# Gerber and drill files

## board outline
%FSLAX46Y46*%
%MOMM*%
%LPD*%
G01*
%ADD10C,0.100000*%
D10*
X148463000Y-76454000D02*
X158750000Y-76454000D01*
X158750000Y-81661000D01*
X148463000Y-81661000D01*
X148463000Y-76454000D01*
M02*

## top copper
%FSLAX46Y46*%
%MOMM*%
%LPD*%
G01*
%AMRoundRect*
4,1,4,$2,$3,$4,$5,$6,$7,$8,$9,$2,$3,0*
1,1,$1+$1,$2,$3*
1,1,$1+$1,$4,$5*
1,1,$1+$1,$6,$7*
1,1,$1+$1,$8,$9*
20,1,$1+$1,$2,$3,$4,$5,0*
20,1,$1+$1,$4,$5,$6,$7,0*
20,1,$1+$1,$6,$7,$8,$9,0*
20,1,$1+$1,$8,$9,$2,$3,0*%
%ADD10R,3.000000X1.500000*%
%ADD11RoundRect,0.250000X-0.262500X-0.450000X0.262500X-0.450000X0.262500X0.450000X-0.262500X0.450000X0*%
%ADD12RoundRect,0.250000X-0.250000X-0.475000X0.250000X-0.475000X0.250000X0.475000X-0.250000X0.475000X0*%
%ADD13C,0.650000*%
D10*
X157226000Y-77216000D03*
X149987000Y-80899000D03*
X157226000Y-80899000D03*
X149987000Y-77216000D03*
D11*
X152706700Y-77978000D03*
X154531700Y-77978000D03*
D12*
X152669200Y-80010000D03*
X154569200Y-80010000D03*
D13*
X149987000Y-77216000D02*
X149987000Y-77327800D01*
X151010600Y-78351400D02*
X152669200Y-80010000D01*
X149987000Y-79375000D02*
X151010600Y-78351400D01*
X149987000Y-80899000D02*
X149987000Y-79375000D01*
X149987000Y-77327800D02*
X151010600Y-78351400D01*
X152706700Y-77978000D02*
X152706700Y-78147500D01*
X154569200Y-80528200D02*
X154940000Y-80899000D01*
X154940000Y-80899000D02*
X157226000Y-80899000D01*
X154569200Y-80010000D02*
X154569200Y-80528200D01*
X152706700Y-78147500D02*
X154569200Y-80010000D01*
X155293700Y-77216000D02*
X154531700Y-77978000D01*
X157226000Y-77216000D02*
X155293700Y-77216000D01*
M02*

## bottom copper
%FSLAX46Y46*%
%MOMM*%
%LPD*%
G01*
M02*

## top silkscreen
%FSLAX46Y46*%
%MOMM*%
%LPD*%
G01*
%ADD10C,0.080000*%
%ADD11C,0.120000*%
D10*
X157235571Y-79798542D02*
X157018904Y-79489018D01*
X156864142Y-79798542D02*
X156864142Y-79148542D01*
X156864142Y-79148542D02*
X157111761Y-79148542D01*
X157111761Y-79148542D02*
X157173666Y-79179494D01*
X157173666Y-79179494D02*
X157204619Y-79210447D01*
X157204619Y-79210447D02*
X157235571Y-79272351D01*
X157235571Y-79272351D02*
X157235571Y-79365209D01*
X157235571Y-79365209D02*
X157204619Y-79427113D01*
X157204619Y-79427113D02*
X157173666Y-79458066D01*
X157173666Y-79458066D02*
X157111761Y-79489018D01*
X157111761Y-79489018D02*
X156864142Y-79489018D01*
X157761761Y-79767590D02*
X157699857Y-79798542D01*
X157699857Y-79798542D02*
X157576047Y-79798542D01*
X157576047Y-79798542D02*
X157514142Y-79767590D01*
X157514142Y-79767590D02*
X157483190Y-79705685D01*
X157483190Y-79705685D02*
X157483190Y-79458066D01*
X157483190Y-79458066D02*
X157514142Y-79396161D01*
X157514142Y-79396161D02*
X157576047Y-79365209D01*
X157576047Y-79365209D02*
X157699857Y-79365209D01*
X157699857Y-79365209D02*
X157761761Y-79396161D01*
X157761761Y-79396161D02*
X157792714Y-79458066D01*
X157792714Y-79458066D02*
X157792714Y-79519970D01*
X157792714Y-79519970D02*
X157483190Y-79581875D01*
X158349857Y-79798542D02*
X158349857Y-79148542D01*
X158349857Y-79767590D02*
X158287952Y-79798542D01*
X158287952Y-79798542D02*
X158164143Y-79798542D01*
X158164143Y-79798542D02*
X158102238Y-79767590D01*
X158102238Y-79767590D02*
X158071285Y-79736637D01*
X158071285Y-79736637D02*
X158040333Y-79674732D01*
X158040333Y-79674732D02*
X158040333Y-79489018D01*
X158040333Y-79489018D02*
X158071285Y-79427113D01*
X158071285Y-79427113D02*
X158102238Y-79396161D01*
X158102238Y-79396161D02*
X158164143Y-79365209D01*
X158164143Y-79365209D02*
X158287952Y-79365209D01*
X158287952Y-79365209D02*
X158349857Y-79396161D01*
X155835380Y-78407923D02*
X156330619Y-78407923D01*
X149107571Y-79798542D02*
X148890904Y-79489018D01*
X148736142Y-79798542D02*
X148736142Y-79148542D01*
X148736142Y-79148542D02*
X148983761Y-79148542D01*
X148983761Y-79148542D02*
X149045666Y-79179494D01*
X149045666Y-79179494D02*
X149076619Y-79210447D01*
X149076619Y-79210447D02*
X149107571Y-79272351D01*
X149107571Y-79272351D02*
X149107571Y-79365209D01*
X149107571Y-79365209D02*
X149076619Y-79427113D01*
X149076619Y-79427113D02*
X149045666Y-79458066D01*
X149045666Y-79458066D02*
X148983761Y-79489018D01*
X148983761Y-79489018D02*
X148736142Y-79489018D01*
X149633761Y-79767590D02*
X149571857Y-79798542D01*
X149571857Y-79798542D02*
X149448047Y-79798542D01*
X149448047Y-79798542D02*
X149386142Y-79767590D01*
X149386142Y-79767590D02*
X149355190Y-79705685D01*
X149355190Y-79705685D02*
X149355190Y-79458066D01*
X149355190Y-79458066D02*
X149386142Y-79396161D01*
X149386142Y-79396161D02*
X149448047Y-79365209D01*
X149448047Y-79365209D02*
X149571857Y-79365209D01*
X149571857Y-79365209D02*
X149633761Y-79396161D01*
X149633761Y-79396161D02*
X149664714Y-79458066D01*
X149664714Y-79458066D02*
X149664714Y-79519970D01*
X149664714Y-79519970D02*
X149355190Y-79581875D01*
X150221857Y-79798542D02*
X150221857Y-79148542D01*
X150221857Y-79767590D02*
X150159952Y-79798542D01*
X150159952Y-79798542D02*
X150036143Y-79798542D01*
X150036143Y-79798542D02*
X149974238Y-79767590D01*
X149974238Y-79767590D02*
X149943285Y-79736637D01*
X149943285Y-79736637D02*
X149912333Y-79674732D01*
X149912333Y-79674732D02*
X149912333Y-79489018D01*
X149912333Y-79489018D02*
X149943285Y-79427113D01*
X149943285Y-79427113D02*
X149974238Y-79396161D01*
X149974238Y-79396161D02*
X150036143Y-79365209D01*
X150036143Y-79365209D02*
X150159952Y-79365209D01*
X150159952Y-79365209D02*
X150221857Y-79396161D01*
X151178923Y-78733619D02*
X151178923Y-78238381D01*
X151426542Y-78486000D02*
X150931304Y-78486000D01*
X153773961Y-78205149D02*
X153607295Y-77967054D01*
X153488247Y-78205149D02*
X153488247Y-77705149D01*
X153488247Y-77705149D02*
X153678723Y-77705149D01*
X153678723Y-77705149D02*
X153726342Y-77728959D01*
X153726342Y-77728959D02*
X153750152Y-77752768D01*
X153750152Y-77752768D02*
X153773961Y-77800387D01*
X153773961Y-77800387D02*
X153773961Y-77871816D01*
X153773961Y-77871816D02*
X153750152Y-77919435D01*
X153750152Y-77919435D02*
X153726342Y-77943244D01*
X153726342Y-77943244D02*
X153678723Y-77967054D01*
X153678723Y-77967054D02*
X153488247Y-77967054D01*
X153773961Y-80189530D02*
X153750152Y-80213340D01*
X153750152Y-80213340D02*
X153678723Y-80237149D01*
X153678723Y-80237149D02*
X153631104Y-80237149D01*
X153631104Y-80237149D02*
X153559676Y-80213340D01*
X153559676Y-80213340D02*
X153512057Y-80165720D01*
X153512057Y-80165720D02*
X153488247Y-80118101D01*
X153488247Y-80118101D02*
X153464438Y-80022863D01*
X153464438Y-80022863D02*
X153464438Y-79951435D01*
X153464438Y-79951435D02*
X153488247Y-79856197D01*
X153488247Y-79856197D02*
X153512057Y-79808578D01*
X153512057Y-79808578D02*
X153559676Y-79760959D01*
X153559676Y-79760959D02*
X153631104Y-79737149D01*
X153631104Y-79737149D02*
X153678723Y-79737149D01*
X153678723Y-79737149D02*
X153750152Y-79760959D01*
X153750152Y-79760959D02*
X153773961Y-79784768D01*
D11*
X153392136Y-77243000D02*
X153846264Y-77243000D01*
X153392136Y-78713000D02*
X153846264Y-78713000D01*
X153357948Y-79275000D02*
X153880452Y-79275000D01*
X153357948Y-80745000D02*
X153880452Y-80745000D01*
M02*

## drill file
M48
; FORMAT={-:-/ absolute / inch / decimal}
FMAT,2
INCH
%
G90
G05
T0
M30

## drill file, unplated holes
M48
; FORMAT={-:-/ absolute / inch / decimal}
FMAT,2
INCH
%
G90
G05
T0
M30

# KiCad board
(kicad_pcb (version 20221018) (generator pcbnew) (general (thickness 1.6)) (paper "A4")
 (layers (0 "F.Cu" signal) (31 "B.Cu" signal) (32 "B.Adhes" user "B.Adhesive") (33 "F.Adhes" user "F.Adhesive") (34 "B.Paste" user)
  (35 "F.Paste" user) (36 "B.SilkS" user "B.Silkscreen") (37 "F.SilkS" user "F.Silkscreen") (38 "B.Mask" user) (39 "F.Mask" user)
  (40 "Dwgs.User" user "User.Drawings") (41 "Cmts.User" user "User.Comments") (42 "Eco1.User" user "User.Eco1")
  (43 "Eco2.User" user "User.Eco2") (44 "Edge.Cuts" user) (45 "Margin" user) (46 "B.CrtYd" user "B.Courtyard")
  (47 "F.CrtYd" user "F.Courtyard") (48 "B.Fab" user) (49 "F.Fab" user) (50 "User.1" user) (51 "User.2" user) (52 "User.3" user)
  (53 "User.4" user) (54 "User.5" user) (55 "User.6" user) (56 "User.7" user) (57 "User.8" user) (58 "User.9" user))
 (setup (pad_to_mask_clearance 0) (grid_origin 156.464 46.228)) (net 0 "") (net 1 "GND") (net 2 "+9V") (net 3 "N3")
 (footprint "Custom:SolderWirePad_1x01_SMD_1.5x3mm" (layer "F.Cu") (at 157.226 77.216 90)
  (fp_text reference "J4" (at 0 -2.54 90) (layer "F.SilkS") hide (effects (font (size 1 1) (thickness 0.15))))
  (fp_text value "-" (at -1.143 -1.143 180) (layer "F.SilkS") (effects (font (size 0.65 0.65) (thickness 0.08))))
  (pad "1" smd rect (at 0 0 90) (size 1.5 3) (layers "F.Cu" "F.Paste" "F.Mask") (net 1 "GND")))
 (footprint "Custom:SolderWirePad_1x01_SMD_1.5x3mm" (layer "F.Cu") (at 149.987 80.899 90)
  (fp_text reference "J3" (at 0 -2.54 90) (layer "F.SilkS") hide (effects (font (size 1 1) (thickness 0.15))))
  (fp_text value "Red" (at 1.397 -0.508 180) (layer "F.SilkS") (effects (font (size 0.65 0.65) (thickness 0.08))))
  (pad "1" smd rect (at 0 0 90) (size 1.5 3) (layers "F.Cu" "F.Paste" "F.Mask") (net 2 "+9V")))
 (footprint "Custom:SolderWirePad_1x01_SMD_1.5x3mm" (layer "F.Cu") (at 157.226 80.899 -90)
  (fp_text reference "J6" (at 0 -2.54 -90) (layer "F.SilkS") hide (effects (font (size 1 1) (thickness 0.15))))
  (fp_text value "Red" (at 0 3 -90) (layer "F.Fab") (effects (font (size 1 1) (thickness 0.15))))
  (pad "1" smd rect (at 0 0 270) (size 1.5 3) (layers "F.Cu" "F.Paste" "F.Mask") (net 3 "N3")))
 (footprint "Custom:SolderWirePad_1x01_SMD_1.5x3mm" (layer "F.Cu") (at 149.987 77.216 -90)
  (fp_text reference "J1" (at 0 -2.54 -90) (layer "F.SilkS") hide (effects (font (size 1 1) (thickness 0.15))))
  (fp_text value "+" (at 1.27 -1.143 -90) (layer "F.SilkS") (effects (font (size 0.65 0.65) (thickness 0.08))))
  (pad "1" smd rect (at 0 0 270) (size 1.5 3) (layers "F.Cu" "F.Paste" "F.Mask") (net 2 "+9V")))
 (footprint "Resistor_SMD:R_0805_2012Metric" (layer "F.Cu") (at 153.6192 77.978)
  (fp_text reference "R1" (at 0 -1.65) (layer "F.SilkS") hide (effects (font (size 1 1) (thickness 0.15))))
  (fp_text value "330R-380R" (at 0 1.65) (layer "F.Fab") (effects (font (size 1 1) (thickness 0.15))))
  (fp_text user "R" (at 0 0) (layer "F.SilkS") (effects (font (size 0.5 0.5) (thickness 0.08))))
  (fp_line (start -0.227064 -0.735) (end 0.227064 -0.735) (stroke (width 0.12) (type solid)) (layer "F.SilkS"))
  (fp_line (start -0.227064 0.735) (end 0.227064 0.735) (stroke (width 0.12) (type solid)) (layer "F.SilkS"))
  (pad "1" smd roundrect (at -0.9125 0) (size 1.025 1.4) (layers "F.Cu" "F.Paste" "F.Mask") (roundrect_rratio 0.243902439) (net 3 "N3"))
  (pad "2" smd roundrect (at 0.9125 0) (size 1.025 1.4) (layers "F.Cu" "F.Paste" "F.Mask") (roundrect_rratio 0.243902439) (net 1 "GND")))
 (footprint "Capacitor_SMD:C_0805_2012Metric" (layer "F.Cu") (at 153.6192 80.01)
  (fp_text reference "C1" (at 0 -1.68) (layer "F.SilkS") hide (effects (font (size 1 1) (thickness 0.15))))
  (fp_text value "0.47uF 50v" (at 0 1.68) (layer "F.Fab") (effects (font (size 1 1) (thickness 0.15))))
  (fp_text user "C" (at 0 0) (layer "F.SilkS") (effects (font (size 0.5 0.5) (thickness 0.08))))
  (fp_line (start -0.261252 -0.735) (end 0.261252 -0.735) (stroke (width 0.12) (type solid)) (layer "F.SilkS"))
  (fp_line (start -0.261252 0.735) (end 0.261252 0.735) (stroke (width 0.12) (type solid)) (layer "F.SilkS"))
  (pad "1" smd roundrect (at -0.95 0) (size 1 1.45) (layers "F.Cu" "F.Paste" "F.Mask") (roundrect_rratio 0.25) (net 2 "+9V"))
  (pad "2" smd roundrect (at 0.95 0) (size 1 1.45) (layers "F.Cu" "F.Paste" "F.Mask") (roundrect_rratio 0.25) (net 3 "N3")))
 (gr_rect (start 148.463 76.454) (end 158.75 81.661) (stroke (width 0.1) (type default)) (fill none) (layer "Edge.Cuts"))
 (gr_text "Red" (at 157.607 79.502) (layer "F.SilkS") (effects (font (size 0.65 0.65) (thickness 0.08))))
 (segment (start 149.987 77.216) (end 149.987 77.3278) (width 0.65) (layer "F.Cu") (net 2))
 (segment (start 151.0106 78.3514) (end 152.6692 80.01) (width 0.65) (layer "F.Cu") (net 2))
 (segment (start 149.987 79.375) (end 151.0106 78.3514) (width 0.65) (layer "F.Cu") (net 2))
 (segment (start 149.987 80.899) (end 149.987 79.375) (width 0.65) (layer "F.Cu") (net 2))
 (segment (start 149.987 77.3278) (end 151.0106 78.3514) (width 0.65) (layer "F.Cu") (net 2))
 (segment (start 152.7067 77.978) (end 152.7067 78.1475) (width 0.65) (layer "F.Cu") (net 3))
 (segment (start 154.5692 80.5282) (end 154.94 80.899) (width 0.65) (layer "F.Cu") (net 3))
 (segment (start 154.94 80.899) (end 157.226 80.899) (width 0.65) (layer "F.Cu") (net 3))
 (segment (start 154.5692 80.01) (end 154.5692 80.5282) (width 0.65) (layer "F.Cu") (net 3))
 (segment (start 152.7067 78.1475) (end 154.5692 80.01) (width 0.65) (layer "F.Cu") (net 3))
 (segment (start 155.2937 77.216) (end 154.5317 77.978) (width 0.65) (layer "F.Cu") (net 1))
 (segment (start 157.226 77.216) (end 155.2937 77.216) (width 0.65) (layer "F.Cu") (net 1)))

